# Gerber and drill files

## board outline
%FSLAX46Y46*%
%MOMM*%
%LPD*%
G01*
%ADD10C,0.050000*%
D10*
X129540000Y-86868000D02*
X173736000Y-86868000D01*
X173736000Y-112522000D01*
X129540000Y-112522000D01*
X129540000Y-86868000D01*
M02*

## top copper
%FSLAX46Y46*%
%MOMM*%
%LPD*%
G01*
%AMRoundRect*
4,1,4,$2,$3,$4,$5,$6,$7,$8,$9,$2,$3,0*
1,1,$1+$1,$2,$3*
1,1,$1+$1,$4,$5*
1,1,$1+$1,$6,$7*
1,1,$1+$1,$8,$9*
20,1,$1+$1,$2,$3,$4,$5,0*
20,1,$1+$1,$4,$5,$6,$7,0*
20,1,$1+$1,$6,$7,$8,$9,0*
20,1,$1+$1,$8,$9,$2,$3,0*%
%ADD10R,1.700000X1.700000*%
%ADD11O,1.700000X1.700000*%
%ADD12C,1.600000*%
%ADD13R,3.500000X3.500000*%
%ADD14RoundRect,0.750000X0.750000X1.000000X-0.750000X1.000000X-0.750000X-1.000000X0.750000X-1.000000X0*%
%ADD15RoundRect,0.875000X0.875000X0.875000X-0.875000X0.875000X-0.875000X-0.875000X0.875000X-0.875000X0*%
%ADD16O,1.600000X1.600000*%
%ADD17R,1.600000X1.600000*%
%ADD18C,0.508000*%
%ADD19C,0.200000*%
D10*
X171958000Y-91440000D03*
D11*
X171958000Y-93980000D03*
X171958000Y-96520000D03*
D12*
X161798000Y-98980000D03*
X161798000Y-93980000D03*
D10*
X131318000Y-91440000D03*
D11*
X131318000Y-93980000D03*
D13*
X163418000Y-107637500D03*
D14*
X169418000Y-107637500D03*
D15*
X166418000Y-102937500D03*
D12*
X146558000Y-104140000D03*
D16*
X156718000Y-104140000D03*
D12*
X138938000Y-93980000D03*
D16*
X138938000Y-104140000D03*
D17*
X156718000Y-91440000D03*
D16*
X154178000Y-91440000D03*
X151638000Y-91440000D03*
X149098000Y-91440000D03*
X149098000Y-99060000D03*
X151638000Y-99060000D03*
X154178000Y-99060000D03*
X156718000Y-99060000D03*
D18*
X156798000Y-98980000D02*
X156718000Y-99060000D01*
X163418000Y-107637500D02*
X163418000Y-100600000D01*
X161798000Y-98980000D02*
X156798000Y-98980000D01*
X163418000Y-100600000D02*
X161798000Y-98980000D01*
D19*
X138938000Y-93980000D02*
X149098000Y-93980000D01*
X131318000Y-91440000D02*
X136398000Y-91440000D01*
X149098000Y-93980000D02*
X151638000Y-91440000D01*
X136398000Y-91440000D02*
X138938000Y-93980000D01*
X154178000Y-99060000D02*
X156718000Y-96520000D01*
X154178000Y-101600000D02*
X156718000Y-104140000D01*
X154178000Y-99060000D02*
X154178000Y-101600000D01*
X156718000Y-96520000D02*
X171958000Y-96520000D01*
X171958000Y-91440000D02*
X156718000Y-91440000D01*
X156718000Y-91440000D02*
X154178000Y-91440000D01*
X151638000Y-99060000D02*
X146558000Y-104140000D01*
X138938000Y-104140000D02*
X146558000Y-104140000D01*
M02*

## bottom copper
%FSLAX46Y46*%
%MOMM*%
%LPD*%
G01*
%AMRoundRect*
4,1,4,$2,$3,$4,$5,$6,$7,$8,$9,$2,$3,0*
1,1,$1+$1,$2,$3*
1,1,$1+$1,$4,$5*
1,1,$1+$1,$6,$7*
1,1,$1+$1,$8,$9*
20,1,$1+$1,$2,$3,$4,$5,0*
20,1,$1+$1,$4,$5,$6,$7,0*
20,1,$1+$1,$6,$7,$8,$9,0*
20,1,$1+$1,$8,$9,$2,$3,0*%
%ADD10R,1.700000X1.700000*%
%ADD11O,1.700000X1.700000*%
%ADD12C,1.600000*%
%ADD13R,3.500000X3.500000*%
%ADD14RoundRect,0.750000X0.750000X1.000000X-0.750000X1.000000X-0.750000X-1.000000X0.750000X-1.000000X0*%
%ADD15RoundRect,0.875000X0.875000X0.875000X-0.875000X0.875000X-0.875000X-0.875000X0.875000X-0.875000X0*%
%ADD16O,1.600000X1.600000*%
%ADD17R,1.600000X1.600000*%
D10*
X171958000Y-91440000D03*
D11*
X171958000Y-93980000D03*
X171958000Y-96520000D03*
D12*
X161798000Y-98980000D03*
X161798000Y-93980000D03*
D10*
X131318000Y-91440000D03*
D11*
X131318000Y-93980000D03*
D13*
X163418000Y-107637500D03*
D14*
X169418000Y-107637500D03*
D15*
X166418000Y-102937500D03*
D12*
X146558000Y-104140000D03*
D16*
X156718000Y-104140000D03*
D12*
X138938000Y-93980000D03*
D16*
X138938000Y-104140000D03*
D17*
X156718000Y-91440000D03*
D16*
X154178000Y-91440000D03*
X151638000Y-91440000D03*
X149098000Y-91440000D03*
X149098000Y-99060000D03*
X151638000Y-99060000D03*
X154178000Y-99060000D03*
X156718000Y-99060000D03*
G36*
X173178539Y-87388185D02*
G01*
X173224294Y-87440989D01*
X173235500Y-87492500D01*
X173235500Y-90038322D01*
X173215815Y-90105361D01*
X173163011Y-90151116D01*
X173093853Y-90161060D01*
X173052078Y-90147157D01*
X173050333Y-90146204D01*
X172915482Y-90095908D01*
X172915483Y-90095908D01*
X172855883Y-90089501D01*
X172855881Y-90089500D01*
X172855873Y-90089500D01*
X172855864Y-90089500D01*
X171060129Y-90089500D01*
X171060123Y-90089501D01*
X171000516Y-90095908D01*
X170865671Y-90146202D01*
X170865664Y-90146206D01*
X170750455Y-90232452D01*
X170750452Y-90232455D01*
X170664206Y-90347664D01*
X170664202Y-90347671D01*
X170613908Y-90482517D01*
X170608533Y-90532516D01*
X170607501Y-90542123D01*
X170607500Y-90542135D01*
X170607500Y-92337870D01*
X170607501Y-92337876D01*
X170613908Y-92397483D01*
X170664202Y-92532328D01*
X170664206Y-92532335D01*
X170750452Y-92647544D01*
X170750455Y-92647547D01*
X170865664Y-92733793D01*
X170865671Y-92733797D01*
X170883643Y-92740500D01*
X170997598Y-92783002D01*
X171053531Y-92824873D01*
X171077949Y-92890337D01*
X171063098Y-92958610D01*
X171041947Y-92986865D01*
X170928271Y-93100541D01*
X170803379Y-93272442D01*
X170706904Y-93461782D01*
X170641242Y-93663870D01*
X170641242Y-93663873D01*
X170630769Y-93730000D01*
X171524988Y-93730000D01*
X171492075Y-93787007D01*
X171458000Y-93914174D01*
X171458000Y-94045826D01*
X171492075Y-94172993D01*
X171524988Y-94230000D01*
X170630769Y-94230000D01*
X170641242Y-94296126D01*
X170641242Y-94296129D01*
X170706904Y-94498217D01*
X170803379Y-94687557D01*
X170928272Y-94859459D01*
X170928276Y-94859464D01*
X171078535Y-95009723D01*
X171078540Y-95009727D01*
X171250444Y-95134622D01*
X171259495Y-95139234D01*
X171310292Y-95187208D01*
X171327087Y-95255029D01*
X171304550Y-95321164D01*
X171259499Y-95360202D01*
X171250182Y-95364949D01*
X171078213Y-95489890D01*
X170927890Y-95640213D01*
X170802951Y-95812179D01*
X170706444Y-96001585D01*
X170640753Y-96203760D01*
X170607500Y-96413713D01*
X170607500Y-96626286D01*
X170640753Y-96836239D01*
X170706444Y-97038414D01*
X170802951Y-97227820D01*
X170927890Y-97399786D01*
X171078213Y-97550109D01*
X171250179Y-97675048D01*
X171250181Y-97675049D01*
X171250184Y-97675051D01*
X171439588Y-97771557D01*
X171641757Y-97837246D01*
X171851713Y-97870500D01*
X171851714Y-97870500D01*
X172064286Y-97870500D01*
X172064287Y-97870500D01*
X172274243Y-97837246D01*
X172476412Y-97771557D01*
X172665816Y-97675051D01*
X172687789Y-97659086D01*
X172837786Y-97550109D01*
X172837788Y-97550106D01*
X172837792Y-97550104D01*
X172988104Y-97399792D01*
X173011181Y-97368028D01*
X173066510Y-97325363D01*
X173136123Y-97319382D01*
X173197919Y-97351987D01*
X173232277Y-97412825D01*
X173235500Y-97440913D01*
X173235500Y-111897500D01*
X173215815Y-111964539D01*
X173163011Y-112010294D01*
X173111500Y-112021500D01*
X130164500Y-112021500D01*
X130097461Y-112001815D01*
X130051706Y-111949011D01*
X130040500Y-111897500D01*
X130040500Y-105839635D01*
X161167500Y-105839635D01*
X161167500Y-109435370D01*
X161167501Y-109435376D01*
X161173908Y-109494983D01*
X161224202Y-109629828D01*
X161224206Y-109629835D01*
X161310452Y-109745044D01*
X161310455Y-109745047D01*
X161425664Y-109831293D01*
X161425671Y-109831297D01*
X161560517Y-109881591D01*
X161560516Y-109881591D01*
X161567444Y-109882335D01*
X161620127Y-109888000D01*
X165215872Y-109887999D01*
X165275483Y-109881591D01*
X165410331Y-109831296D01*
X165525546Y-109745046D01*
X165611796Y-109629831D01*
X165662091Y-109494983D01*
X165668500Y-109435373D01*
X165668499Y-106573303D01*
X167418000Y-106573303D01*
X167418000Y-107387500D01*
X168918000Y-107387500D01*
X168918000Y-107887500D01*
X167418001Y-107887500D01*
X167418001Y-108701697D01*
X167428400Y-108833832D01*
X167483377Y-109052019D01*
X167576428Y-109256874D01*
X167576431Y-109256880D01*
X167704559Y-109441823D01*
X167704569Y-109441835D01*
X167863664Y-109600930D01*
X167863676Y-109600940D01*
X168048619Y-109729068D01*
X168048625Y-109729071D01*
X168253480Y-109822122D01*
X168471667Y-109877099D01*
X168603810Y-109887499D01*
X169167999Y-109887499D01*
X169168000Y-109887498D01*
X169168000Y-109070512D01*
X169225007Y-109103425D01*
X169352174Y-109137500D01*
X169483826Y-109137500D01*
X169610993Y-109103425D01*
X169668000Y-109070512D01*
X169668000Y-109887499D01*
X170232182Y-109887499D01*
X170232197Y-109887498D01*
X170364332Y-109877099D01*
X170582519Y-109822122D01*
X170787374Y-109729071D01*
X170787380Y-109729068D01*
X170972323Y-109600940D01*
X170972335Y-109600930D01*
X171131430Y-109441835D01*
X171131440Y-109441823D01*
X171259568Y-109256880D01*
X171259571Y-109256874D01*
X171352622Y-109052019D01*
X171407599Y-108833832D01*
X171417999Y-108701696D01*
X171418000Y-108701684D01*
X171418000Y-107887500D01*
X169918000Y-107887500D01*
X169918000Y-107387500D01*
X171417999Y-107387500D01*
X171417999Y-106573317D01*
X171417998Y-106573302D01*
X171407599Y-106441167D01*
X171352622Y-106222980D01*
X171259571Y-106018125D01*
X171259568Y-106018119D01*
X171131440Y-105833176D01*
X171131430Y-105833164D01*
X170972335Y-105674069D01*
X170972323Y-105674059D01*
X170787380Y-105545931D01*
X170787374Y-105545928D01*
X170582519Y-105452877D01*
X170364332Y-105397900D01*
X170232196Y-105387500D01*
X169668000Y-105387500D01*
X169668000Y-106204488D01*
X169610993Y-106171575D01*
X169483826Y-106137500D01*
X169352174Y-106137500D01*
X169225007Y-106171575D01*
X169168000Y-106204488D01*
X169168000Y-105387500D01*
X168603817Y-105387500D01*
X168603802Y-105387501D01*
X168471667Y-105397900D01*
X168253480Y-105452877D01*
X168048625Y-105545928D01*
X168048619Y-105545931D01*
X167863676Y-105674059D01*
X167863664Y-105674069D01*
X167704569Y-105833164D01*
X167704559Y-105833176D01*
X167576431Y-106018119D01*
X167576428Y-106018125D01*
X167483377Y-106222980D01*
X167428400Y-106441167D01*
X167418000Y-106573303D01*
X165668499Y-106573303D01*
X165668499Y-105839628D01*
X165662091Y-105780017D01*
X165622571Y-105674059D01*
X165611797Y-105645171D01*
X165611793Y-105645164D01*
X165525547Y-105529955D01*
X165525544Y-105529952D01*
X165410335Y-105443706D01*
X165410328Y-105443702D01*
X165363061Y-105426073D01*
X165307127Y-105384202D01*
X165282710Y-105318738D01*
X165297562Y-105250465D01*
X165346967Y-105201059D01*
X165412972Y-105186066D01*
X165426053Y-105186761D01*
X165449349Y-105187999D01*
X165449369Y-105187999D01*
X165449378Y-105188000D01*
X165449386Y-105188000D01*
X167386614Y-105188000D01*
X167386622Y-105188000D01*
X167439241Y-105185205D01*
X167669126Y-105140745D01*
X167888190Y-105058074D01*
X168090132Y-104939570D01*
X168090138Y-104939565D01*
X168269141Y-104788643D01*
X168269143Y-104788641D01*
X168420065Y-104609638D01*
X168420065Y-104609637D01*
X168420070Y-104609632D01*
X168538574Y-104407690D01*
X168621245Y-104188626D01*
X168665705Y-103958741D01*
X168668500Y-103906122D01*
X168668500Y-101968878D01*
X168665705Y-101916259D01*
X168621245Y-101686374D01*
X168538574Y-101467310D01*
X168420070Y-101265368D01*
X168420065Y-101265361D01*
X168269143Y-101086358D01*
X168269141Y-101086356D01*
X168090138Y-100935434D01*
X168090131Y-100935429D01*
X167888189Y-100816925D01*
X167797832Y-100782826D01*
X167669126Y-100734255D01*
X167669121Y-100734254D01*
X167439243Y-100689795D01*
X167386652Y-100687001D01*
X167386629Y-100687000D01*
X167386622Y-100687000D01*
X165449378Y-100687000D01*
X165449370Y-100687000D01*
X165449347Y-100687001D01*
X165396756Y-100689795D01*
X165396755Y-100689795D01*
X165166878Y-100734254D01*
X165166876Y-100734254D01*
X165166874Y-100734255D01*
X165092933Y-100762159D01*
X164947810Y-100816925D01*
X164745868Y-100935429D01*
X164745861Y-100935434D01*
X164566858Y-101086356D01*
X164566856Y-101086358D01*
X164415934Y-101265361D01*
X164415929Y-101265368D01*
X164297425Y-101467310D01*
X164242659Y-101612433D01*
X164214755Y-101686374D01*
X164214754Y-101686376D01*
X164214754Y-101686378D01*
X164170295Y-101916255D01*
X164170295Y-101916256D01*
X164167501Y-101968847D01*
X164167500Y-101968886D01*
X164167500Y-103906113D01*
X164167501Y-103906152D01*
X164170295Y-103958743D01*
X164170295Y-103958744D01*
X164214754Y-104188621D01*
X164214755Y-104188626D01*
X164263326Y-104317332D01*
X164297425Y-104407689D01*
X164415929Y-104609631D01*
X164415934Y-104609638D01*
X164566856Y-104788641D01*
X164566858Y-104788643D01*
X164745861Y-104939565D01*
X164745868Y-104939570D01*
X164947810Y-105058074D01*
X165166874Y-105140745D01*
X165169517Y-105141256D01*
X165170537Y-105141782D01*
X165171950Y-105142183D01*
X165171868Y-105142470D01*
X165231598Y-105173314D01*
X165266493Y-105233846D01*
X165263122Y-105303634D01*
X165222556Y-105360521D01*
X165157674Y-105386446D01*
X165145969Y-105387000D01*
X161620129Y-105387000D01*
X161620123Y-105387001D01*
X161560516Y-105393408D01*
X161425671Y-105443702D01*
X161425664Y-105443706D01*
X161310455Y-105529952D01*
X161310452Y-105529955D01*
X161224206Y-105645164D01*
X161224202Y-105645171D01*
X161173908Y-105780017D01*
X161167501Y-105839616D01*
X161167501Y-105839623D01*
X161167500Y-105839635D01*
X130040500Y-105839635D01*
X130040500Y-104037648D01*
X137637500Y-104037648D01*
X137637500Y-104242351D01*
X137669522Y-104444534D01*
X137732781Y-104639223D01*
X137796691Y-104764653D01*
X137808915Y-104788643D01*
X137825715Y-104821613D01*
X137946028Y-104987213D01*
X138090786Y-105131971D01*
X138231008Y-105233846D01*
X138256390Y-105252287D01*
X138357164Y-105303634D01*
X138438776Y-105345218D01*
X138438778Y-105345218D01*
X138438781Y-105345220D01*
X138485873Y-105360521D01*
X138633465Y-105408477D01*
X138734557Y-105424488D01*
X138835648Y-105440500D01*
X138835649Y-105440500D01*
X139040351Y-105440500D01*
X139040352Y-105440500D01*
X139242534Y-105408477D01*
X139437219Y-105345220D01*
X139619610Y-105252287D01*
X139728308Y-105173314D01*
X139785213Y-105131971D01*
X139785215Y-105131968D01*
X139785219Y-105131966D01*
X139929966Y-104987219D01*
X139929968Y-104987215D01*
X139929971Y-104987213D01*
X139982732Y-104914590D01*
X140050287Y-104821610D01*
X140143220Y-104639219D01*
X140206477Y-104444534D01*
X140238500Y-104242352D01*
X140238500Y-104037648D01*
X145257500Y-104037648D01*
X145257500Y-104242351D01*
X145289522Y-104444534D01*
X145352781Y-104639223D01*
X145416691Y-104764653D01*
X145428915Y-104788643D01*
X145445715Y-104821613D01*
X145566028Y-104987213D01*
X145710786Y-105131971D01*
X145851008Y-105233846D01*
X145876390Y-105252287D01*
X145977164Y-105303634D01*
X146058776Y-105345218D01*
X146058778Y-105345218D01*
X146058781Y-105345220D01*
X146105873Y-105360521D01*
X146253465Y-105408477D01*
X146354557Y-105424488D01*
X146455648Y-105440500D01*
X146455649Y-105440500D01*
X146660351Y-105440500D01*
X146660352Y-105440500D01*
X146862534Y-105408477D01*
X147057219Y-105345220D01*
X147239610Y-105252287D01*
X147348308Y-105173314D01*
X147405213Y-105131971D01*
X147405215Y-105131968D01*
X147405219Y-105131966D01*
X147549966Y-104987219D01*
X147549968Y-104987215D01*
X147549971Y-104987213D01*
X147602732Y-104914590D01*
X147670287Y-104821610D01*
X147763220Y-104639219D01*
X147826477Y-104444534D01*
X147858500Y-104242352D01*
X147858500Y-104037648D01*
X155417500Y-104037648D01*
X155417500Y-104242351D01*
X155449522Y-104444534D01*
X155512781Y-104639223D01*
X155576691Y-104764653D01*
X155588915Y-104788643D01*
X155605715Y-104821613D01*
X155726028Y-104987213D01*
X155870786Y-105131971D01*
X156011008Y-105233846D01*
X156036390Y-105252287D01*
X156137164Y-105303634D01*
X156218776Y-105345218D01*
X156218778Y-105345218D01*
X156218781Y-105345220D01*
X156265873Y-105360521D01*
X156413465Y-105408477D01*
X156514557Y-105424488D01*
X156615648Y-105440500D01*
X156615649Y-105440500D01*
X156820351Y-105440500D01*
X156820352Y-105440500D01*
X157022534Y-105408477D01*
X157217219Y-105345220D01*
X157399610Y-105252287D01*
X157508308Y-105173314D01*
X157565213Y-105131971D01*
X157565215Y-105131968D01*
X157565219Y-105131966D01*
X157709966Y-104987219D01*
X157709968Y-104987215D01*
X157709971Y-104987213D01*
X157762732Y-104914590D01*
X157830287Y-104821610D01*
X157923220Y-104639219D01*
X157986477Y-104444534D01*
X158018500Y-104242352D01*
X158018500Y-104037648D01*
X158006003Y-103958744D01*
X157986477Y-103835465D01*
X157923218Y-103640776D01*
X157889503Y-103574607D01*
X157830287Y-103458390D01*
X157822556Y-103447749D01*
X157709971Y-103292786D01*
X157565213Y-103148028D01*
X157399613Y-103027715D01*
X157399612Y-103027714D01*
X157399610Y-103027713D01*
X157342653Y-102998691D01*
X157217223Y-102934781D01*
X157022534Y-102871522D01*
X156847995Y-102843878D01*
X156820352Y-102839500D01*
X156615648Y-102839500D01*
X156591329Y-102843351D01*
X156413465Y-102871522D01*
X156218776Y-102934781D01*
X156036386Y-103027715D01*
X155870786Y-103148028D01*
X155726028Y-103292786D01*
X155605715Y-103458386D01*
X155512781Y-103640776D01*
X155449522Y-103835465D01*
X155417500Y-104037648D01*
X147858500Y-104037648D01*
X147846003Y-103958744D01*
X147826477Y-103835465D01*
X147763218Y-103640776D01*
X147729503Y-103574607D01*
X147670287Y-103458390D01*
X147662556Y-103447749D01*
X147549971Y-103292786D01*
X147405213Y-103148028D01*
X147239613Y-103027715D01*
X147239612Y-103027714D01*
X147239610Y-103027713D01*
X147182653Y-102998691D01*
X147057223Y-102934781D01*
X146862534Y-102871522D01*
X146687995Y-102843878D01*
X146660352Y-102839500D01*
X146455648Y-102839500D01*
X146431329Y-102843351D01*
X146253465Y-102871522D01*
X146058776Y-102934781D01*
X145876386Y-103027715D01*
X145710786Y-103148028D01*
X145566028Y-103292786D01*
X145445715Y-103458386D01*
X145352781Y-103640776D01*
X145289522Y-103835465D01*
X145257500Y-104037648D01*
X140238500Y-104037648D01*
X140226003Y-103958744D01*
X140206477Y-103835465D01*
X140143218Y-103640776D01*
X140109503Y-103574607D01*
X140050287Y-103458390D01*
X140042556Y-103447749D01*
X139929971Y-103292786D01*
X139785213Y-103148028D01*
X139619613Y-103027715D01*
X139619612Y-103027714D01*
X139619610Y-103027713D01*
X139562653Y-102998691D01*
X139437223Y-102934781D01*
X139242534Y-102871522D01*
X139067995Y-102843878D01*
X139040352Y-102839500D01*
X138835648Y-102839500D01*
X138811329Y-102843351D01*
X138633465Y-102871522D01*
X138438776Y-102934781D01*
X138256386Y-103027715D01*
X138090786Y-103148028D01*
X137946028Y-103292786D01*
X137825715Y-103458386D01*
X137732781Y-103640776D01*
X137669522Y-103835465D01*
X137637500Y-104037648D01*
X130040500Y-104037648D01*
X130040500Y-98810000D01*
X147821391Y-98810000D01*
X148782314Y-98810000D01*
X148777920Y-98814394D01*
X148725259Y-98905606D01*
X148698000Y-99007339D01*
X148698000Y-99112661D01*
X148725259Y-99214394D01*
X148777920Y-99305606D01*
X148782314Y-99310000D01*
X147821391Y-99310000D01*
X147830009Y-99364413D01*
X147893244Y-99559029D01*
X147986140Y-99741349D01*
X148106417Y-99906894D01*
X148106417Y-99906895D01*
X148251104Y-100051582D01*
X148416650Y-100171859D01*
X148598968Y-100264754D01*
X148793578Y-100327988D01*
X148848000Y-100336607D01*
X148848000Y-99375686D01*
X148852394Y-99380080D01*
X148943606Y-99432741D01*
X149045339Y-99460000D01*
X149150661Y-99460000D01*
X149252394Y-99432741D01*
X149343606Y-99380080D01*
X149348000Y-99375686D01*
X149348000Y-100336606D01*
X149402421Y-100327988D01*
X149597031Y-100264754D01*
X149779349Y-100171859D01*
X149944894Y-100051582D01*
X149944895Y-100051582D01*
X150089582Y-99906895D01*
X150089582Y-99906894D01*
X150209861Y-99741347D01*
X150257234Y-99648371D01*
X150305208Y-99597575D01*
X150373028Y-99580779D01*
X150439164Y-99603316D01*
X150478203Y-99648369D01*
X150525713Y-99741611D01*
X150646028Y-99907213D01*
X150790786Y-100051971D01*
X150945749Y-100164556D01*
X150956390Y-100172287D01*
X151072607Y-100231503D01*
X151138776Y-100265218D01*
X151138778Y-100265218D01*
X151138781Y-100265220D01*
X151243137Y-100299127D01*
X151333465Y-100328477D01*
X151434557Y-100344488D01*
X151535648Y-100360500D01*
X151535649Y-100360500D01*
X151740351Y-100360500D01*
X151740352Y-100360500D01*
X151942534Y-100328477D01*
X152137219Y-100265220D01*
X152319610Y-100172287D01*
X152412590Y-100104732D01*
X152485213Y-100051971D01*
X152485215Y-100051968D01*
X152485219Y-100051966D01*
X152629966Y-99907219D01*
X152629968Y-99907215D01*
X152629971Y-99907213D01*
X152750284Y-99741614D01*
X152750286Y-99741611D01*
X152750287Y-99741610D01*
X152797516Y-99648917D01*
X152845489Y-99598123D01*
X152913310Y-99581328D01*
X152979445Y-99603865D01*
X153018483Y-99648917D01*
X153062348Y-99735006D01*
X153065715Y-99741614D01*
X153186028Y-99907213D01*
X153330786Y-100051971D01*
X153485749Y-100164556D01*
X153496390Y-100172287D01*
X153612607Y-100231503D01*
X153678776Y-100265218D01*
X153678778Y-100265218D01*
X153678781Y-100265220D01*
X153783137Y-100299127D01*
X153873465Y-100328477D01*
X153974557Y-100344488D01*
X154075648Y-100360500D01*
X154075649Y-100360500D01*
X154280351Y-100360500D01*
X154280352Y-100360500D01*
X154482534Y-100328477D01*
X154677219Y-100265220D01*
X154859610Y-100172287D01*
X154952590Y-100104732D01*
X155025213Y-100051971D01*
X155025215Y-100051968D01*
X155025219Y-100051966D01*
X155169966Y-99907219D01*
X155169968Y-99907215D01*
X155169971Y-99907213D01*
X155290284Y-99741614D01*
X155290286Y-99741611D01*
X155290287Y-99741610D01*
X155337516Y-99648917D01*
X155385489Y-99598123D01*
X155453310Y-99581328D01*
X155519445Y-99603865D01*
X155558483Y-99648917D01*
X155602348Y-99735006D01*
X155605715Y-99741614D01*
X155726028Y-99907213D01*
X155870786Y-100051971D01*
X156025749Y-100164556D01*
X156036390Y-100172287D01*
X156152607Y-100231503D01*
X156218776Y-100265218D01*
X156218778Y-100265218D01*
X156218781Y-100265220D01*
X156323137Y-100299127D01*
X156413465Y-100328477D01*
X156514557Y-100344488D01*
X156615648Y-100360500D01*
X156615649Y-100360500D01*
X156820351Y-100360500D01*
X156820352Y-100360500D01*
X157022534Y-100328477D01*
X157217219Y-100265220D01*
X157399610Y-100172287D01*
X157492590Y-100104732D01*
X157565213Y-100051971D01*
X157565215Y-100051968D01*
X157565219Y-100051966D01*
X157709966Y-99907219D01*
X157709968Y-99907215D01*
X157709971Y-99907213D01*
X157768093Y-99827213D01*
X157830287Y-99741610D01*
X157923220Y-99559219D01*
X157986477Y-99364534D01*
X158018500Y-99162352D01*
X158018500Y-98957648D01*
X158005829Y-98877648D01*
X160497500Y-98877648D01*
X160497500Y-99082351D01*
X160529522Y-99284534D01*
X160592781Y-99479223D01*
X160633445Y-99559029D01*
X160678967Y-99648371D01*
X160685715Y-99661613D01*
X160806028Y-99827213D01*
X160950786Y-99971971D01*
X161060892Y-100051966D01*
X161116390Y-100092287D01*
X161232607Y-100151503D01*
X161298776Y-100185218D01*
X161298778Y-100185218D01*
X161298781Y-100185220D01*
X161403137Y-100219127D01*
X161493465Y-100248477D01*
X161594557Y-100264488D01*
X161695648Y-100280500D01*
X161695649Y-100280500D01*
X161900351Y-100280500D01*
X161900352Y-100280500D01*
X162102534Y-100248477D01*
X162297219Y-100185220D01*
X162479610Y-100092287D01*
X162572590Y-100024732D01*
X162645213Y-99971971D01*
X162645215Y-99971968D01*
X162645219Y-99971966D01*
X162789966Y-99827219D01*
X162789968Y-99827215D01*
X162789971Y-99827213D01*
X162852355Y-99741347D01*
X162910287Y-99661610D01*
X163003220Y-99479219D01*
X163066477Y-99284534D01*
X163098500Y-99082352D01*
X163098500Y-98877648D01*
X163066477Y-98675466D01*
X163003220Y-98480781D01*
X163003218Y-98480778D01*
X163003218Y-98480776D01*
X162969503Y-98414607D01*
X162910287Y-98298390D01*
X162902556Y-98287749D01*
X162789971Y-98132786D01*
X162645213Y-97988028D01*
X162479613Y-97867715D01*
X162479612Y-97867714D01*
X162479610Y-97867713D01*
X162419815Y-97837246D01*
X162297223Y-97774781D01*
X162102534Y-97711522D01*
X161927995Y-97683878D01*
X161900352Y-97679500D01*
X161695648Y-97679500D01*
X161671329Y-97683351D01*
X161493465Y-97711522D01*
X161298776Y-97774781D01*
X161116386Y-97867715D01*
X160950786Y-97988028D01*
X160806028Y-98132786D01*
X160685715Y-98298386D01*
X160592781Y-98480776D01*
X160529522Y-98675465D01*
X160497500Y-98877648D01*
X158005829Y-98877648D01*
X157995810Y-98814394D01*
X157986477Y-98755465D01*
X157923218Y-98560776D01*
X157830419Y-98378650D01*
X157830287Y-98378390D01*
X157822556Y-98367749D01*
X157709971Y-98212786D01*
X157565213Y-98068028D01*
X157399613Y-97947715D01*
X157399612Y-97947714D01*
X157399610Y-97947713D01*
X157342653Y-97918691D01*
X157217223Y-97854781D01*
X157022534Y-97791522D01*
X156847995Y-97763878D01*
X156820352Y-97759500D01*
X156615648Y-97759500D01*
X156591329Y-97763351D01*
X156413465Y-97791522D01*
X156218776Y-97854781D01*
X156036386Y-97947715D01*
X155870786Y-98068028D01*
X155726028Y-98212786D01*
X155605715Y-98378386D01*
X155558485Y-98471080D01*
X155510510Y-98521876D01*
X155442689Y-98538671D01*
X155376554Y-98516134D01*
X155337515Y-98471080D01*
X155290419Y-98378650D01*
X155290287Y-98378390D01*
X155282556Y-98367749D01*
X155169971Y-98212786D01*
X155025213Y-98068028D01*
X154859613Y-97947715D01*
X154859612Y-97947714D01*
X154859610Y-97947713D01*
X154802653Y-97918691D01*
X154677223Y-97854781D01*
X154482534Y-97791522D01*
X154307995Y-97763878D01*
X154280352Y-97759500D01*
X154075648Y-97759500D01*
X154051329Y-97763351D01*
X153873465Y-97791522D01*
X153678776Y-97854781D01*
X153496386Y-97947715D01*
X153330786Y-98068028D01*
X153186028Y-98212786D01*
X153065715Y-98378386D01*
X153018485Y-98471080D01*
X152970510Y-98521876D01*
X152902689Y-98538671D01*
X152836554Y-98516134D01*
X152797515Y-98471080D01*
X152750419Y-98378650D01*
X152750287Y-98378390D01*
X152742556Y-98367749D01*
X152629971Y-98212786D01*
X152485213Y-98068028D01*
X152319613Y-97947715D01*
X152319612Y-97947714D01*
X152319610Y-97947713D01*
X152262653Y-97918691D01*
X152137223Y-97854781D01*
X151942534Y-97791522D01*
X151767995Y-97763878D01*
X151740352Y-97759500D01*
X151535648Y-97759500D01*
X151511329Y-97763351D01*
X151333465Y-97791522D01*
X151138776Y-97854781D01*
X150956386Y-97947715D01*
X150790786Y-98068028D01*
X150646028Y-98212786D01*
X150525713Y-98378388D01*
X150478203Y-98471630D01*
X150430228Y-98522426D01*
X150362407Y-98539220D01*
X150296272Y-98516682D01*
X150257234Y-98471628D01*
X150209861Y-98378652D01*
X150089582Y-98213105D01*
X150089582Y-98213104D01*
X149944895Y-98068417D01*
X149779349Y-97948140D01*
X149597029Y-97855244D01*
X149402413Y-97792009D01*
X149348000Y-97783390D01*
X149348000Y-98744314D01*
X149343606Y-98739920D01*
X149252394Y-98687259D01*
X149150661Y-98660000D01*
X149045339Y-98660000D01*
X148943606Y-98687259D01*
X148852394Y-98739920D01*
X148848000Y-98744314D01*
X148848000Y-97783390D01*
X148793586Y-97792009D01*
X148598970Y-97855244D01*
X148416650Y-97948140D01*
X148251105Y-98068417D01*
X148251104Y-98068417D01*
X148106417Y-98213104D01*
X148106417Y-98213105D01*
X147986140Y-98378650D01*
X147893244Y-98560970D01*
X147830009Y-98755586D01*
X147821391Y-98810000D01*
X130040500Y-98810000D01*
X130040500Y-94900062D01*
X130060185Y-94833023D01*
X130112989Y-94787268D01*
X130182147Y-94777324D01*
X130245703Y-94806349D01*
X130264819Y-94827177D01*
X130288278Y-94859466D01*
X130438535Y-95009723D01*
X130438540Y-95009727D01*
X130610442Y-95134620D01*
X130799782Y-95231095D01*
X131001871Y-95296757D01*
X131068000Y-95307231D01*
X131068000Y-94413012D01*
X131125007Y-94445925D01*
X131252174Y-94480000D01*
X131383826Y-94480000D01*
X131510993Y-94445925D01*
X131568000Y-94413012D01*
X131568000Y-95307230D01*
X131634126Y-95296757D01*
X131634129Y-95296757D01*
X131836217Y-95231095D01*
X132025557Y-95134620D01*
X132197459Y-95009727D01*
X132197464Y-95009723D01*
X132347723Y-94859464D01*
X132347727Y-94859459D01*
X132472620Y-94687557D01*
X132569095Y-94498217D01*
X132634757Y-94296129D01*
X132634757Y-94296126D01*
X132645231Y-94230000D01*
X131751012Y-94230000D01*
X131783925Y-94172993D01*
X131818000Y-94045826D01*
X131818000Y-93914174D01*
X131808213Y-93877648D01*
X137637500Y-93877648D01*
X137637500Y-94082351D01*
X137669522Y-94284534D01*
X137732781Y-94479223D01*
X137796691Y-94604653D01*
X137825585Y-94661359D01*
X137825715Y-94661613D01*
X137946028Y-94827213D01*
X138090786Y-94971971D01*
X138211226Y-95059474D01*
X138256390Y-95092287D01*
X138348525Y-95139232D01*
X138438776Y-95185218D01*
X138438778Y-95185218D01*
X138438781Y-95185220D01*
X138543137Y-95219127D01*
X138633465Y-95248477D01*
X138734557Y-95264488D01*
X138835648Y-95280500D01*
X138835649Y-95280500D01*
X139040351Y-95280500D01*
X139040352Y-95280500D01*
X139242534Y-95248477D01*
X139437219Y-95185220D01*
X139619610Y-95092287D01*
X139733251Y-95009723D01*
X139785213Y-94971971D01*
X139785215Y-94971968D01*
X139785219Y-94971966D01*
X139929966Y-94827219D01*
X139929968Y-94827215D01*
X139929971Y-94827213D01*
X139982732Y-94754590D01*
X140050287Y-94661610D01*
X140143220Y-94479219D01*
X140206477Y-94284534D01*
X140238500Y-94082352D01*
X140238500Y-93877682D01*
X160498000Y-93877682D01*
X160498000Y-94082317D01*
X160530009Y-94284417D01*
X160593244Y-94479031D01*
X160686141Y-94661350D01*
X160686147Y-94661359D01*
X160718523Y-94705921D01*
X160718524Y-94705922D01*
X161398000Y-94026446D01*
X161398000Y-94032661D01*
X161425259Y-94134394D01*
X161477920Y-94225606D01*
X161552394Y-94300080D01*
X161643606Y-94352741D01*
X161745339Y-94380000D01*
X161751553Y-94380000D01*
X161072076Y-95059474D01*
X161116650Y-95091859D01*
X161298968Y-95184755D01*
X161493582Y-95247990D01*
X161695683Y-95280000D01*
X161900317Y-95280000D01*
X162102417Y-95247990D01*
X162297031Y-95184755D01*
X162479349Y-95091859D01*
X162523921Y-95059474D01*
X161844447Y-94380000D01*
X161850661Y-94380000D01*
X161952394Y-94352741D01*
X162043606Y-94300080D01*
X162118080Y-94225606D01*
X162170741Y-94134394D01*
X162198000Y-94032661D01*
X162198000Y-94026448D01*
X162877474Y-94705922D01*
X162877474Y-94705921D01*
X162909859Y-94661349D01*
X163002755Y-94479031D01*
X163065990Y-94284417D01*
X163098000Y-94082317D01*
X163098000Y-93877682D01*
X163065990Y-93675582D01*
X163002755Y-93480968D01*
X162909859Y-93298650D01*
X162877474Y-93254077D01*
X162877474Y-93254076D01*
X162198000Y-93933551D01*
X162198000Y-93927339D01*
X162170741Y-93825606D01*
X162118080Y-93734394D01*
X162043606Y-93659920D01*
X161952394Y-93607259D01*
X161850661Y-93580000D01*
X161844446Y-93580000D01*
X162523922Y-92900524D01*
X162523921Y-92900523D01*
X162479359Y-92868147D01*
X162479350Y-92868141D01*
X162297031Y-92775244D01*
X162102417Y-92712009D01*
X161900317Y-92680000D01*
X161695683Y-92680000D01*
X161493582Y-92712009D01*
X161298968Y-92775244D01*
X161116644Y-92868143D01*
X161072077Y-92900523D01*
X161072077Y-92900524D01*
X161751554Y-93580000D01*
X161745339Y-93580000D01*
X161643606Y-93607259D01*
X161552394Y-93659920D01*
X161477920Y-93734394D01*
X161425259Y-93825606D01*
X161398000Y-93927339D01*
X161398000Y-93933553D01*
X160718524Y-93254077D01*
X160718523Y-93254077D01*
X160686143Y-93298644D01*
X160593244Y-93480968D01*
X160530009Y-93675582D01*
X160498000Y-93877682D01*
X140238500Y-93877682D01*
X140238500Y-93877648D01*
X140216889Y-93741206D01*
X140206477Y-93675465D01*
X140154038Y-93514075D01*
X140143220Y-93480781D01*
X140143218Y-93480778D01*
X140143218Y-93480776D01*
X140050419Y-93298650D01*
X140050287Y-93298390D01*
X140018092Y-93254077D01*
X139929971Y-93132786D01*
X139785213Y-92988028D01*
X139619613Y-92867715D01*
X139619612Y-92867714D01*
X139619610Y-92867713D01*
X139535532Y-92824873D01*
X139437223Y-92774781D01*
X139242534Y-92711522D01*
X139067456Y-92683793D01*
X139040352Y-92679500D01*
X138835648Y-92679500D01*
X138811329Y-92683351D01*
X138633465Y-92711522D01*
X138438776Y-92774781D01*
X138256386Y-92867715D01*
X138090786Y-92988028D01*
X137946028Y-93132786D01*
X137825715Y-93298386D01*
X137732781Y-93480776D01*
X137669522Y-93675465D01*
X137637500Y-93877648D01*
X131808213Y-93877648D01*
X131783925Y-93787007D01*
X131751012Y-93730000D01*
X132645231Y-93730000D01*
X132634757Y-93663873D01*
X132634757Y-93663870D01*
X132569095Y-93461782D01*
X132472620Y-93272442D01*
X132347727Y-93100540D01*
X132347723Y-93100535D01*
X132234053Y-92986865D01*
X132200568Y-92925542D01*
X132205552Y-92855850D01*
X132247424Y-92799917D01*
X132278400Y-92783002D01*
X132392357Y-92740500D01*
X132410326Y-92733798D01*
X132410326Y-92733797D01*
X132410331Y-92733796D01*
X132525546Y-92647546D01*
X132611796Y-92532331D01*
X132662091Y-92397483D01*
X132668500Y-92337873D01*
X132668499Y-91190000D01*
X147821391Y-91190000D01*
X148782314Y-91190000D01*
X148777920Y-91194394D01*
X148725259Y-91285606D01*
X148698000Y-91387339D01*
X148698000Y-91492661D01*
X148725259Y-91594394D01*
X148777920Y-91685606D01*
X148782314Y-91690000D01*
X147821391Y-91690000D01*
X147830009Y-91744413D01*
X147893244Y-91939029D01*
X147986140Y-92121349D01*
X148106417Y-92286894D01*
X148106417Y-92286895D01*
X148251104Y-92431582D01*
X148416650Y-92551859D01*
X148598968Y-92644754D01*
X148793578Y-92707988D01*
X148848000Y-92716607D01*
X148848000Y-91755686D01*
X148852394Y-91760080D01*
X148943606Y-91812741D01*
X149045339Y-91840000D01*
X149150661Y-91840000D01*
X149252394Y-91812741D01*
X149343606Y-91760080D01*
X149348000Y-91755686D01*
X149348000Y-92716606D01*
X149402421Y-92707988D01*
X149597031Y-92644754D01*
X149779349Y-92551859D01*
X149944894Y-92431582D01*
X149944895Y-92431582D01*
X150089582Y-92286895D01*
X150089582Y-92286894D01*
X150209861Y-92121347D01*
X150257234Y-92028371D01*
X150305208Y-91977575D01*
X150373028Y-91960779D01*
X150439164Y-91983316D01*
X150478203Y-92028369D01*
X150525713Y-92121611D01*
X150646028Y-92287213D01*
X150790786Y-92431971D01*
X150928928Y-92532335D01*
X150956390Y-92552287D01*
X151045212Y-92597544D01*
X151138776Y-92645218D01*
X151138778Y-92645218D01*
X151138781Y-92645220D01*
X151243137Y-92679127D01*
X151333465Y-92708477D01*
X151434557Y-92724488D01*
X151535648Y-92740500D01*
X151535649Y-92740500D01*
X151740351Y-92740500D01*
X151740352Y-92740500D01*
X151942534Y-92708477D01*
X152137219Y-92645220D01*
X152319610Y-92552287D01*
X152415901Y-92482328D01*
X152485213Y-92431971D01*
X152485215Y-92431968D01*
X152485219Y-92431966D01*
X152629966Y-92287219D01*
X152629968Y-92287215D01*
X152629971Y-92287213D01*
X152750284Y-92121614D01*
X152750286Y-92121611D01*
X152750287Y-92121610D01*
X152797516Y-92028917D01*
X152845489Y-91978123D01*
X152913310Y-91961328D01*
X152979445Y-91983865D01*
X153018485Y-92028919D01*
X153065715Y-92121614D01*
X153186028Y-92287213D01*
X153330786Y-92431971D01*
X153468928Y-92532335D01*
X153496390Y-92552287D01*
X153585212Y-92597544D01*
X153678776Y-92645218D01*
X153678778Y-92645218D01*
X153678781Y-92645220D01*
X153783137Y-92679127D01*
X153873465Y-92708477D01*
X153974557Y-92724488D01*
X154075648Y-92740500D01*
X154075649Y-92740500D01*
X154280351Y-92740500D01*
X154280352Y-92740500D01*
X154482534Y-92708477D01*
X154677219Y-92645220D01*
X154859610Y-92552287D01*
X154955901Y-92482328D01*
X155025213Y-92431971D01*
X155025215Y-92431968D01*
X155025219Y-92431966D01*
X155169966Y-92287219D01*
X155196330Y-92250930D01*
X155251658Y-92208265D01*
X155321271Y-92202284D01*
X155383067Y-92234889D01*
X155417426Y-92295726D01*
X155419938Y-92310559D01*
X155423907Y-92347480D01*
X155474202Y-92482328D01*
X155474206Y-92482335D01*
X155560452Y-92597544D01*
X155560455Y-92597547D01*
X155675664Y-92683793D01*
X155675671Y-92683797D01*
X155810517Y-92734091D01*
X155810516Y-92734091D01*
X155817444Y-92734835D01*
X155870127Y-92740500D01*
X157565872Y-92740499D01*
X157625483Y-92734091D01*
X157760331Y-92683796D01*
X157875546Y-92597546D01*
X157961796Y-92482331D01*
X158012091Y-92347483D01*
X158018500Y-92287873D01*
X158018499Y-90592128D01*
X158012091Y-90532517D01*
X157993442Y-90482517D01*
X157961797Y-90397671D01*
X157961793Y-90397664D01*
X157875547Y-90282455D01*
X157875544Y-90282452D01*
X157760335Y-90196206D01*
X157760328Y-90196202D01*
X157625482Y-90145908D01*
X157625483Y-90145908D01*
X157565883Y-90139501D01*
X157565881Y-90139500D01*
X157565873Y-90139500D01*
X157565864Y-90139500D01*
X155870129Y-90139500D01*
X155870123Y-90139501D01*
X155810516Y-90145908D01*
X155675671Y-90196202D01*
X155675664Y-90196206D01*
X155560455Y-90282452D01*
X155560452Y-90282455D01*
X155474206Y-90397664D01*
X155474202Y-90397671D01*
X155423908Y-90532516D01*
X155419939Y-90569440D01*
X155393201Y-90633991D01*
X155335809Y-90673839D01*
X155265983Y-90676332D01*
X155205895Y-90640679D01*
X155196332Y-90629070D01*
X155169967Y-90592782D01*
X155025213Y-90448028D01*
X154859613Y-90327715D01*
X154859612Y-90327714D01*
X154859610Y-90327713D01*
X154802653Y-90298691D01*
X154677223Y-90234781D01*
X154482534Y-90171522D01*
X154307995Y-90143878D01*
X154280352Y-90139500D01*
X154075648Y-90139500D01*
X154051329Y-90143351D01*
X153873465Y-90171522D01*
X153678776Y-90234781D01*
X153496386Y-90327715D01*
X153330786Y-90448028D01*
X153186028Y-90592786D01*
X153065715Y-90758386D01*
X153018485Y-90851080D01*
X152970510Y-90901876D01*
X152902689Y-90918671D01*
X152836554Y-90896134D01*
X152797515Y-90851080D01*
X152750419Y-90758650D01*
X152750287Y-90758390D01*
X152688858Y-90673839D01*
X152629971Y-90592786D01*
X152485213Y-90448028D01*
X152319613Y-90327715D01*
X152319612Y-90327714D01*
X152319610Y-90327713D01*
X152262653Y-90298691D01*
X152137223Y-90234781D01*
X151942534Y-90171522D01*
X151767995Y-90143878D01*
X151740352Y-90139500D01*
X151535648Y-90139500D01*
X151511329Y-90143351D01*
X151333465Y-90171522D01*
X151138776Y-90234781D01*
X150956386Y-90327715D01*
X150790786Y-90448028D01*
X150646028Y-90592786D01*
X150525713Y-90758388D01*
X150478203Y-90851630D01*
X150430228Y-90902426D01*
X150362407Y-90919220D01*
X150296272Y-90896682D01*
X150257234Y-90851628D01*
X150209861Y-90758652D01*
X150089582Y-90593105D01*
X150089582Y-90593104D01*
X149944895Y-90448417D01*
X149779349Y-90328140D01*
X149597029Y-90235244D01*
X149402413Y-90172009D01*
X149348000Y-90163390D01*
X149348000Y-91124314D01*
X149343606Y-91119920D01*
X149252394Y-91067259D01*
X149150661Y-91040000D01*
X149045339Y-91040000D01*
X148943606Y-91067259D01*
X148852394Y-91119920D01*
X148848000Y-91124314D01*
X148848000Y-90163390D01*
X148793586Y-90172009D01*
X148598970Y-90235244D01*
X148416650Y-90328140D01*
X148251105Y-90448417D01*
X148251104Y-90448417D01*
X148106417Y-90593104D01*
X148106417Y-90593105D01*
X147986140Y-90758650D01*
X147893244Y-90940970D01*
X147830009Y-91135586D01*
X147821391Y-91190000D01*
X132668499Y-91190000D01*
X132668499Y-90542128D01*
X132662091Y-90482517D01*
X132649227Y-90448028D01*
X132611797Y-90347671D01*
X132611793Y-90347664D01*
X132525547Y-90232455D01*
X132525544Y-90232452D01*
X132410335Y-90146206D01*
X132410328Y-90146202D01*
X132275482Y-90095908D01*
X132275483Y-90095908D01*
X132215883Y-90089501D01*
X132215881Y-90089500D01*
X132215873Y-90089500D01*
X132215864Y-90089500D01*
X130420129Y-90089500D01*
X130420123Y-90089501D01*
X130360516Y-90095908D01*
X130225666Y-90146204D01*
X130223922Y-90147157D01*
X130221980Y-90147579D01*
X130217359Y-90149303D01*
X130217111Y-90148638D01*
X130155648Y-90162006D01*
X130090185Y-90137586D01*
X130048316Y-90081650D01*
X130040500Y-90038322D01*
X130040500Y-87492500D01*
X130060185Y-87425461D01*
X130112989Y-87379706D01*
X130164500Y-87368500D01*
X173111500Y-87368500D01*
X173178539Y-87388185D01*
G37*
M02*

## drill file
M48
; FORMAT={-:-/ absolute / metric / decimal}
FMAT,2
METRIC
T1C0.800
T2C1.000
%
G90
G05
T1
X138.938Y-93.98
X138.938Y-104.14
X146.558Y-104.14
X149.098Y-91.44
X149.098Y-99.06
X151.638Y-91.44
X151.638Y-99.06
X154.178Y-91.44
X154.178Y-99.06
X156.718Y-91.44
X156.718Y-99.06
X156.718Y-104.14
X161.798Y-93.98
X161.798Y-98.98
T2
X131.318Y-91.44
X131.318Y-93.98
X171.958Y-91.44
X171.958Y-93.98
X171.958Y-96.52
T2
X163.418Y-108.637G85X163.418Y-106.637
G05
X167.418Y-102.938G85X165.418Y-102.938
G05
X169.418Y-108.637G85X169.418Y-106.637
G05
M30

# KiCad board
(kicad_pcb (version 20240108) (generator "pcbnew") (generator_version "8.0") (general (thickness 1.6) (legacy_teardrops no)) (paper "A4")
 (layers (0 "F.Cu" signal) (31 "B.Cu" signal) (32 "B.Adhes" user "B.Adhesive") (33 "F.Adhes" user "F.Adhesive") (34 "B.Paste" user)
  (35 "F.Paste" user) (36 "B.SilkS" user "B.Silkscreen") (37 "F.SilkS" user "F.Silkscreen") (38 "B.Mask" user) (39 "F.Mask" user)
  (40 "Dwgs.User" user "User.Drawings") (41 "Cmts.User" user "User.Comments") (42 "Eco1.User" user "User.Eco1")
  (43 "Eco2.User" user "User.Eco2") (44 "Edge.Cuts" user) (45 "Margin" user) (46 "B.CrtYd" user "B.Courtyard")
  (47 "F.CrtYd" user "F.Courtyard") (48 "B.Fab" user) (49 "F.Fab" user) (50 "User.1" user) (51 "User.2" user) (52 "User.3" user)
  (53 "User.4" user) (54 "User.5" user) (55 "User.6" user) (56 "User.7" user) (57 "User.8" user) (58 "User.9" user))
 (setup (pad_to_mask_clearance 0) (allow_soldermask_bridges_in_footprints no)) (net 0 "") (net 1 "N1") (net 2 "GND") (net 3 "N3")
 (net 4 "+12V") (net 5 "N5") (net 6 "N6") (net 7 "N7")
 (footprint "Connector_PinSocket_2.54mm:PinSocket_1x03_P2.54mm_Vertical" (layer "F.Cu") (at 171.958 91.44)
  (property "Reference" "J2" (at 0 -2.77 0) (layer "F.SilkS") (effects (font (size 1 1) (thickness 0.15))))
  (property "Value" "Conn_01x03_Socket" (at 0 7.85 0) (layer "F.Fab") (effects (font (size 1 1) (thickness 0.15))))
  (pad "1" thru_hole rect (at 0 0) (size 1.7 1.7) (drill 1) (layers "*.Cu" "*.Mask") (remove_unused_layers no) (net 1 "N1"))
  (pad "2" thru_hole oval (at 0 2.54) (size 1.7 1.7) (drill 1) (layers "*.Cu" "*.Mask") (remove_unused_layers no) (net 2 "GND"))
  (pad "3" thru_hole oval (at 0 5.08) (size 1.7 1.7) (drill 1) (layers "*.Cu" "*.Mask") (remove_unused_layers no) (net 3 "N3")))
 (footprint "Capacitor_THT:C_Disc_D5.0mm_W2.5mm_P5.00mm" (layer "F.Cu") (at 161.798 98.98 90)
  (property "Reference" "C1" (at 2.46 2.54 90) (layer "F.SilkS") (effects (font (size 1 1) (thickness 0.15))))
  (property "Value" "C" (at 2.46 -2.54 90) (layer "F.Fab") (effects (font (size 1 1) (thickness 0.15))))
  (pad "1" thru_hole circle (at 0 0 90) (size 1.6 1.6) (drill 0.8) (layers "*.Cu" "*.Mask") (remove_unused_layers no) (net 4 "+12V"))
  (pad "2" thru_hole circle (at 5 0 90) (size 1.6 1.6) (drill 0.8) (layers "*.Cu" "*.Mask") (remove_unused_layers no) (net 2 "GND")))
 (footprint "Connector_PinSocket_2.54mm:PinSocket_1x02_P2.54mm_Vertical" (layer "F.Cu") (at 131.318 91.44)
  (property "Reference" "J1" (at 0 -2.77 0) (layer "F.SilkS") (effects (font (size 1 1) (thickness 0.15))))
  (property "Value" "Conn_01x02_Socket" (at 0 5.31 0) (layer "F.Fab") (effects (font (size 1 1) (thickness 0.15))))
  (pad "1" thru_hole rect (at 0 0) (size 1.7 1.7) (drill 1) (layers "*.Cu" "*.Mask") (remove_unused_layers no) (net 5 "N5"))
  (pad "2" thru_hole oval (at 0 2.54) (size 1.7 1.7) (drill 1) (layers "*.Cu" "*.Mask") (remove_unused_layers no) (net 2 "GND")))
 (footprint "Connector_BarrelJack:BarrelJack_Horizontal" (layer "F.Cu") (at 163.418 107.6375 180)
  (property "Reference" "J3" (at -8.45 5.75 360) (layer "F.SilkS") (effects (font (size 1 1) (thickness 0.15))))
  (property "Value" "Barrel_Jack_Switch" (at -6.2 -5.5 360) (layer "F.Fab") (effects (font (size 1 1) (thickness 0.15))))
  (pad "1" thru_hole rect (at 0 0 180) (size 3.5 3.5) (drill oval 1 3) (layers "*.Cu" "*.Mask") (remove_unused_layers no) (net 4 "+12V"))
  (pad "2" thru_hole roundrect (at -6 0 180) (size 3 3.5) (drill oval 1 3) (layers "*.Cu" "*.Mask") (remove_unused_layers no)
   (roundrect_rratio 0.25) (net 2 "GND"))
  (pad "3" thru_hole roundrect (at -3 4.7 180) (size 3.5 3.5) (drill oval 3 1) (layers "*.Cu" "*.Mask") (remove_unused_layers no)
   (roundrect_rratio 0.25) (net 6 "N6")))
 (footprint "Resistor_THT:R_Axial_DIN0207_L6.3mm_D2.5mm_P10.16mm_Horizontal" (layer "F.Cu") (at 146.558 104.14)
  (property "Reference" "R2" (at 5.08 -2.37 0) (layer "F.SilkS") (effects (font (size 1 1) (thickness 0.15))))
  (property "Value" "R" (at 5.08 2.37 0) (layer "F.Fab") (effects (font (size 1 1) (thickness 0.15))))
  (pad "1" thru_hole circle (at 0 0) (size 1.6 1.6) (drill 0.8) (layers "*.Cu" "*.Mask") (remove_unused_layers no) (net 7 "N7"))
  (pad "2" thru_hole oval (at 10.16 0) (size 1.6 1.6) (drill 0.8) (layers "*.Cu" "*.Mask") (remove_unused_layers no) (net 3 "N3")))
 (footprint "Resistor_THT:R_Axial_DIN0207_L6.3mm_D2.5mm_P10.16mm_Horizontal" (layer "F.Cu") (at 138.938 93.98 -90)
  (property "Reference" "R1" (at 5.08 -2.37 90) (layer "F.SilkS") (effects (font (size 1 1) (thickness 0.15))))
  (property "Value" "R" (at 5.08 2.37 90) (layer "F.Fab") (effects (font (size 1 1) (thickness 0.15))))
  (pad "1" thru_hole circle (at 0 0 270) (size 1.6 1.6) (drill 0.8) (layers "*.Cu" "*.Mask") (remove_unused_layers no) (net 5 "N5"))
  (pad "2" thru_hole oval (at 10.16 0 270) (size 1.6 1.6) (drill 0.8) (layers "*.Cu" "*.Mask") (remove_unused_layers no) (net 7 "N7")))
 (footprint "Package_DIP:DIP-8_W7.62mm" (layer "F.Cu") (at 156.718 91.44 -90)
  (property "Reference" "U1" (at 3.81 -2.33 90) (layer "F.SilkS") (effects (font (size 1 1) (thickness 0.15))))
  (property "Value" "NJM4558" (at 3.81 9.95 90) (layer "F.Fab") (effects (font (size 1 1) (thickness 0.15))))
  (pad "1" thru_hole rect (at 0 0 270) (size 1.6 1.6) (drill 0.8) (layers "*.Cu" "*.Mask") (remove_unused_layers no) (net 1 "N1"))
  (pad "2" thru_hole oval (at 0 2.54 270) (size 1.6 1.6) (drill 0.8) (layers "*.Cu" "*.Mask") (remove_unused_layers no) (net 1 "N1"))
  (pad "3" thru_hole oval (at 0 5.08 270) (size 1.6 1.6) (drill 0.8) (layers "*.Cu" "*.Mask") (remove_unused_layers no) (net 5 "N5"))
  (pad "4" thru_hole oval (at 0 7.62 270) (size 1.6 1.6) (drill 0.8) (layers "*.Cu" "*.Mask") (remove_unused_layers no) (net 2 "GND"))
  (pad "5" thru_hole oval (at 7.62 7.62 270) (size 1.6 1.6) (drill 0.8) (layers "*.Cu" "*.Mask") (remove_unused_layers no) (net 2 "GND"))
  (pad "6" thru_hole oval (at 7.62 5.08 270) (size 1.6 1.6) (drill 0.8) (layers "*.Cu" "*.Mask") (remove_unused_layers no) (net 7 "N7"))
  (pad "7" thru_hole oval (at 7.62 2.54 270) (size 1.6 1.6) (drill 0.8) (layers "*.Cu" "*.Mask") (remove_unused_layers no) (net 3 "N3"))
  (pad "8" thru_hole oval (at 7.62 0 270) (size 1.6 1.6) (drill 0.8) (layers "*.Cu" "*.Mask") (remove_unused_layers no) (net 4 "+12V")))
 (gr_rect (start 129.54 86.868) (end 173.736 112.522) (stroke (width 0.05) (type default)) (fill none) (layer "Edge.Cuts"))
 (segment (start 156.798 98.98) (end 156.718 99.06) (width 0.508) (layer "F.Cu") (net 4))
 (segment (start 163.418 107.6375) (end 163.418 100.6) (width 0.508) (layer "F.Cu") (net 4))
 (segment (start 161.798 98.98) (end 156.798 98.98) (width 0.508) (layer "F.Cu") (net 4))
 (segment (start 163.418 100.6) (end 161.798 98.98) (width 0.508) (layer "F.Cu") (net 4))
 (segment (start 138.938 93.98) (end 149.098 93.98) (width 0.2) (layer "F.Cu") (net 5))
 (segment (start 131.318 91.44) (end 136.398 91.44) (width 0.2) (layer "F.Cu") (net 5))
 (segment (start 149.098 93.98) (end 151.638 91.44) (width 0.2) (layer "F.Cu") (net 5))
 (segment (start 136.398 91.44) (end 138.938 93.98) (width 0.2) (layer "F.Cu") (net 5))
 (segment (start 154.178 99.06) (end 156.718 96.52) (width 0.2) (layer "F.Cu") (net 3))
 (segment (start 154.178 101.6) (end 156.718 104.14) (width 0.2) (layer "F.Cu") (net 3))
 (segment (start 154.178 99.06) (end 154.178 101.6) (width 0.2) (layer "F.Cu") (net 3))
 (segment (start 156.718 96.52) (end 171.958 96.52) (width 0.2) (layer "F.Cu") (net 3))
 (segment (start 171.958 91.44) (end 156.718 91.44) (width 0.2) (layer "F.Cu") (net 1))
 (segment (start 156.718 91.44) (end 154.178 91.44) (width 0.2) (layer "F.Cu") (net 1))
 (segment (start 151.638 99.06) (end 146.558 104.14) (width 0.2) (layer "F.Cu") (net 7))
 (segment (start 138.938 104.14) (end 146.558 104.14) (width 0.2) (layer "F.Cu") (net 7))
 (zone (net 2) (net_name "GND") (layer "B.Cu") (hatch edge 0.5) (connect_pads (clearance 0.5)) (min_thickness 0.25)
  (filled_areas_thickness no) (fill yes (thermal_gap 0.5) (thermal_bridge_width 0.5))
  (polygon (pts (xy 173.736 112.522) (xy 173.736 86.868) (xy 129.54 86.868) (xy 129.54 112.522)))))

